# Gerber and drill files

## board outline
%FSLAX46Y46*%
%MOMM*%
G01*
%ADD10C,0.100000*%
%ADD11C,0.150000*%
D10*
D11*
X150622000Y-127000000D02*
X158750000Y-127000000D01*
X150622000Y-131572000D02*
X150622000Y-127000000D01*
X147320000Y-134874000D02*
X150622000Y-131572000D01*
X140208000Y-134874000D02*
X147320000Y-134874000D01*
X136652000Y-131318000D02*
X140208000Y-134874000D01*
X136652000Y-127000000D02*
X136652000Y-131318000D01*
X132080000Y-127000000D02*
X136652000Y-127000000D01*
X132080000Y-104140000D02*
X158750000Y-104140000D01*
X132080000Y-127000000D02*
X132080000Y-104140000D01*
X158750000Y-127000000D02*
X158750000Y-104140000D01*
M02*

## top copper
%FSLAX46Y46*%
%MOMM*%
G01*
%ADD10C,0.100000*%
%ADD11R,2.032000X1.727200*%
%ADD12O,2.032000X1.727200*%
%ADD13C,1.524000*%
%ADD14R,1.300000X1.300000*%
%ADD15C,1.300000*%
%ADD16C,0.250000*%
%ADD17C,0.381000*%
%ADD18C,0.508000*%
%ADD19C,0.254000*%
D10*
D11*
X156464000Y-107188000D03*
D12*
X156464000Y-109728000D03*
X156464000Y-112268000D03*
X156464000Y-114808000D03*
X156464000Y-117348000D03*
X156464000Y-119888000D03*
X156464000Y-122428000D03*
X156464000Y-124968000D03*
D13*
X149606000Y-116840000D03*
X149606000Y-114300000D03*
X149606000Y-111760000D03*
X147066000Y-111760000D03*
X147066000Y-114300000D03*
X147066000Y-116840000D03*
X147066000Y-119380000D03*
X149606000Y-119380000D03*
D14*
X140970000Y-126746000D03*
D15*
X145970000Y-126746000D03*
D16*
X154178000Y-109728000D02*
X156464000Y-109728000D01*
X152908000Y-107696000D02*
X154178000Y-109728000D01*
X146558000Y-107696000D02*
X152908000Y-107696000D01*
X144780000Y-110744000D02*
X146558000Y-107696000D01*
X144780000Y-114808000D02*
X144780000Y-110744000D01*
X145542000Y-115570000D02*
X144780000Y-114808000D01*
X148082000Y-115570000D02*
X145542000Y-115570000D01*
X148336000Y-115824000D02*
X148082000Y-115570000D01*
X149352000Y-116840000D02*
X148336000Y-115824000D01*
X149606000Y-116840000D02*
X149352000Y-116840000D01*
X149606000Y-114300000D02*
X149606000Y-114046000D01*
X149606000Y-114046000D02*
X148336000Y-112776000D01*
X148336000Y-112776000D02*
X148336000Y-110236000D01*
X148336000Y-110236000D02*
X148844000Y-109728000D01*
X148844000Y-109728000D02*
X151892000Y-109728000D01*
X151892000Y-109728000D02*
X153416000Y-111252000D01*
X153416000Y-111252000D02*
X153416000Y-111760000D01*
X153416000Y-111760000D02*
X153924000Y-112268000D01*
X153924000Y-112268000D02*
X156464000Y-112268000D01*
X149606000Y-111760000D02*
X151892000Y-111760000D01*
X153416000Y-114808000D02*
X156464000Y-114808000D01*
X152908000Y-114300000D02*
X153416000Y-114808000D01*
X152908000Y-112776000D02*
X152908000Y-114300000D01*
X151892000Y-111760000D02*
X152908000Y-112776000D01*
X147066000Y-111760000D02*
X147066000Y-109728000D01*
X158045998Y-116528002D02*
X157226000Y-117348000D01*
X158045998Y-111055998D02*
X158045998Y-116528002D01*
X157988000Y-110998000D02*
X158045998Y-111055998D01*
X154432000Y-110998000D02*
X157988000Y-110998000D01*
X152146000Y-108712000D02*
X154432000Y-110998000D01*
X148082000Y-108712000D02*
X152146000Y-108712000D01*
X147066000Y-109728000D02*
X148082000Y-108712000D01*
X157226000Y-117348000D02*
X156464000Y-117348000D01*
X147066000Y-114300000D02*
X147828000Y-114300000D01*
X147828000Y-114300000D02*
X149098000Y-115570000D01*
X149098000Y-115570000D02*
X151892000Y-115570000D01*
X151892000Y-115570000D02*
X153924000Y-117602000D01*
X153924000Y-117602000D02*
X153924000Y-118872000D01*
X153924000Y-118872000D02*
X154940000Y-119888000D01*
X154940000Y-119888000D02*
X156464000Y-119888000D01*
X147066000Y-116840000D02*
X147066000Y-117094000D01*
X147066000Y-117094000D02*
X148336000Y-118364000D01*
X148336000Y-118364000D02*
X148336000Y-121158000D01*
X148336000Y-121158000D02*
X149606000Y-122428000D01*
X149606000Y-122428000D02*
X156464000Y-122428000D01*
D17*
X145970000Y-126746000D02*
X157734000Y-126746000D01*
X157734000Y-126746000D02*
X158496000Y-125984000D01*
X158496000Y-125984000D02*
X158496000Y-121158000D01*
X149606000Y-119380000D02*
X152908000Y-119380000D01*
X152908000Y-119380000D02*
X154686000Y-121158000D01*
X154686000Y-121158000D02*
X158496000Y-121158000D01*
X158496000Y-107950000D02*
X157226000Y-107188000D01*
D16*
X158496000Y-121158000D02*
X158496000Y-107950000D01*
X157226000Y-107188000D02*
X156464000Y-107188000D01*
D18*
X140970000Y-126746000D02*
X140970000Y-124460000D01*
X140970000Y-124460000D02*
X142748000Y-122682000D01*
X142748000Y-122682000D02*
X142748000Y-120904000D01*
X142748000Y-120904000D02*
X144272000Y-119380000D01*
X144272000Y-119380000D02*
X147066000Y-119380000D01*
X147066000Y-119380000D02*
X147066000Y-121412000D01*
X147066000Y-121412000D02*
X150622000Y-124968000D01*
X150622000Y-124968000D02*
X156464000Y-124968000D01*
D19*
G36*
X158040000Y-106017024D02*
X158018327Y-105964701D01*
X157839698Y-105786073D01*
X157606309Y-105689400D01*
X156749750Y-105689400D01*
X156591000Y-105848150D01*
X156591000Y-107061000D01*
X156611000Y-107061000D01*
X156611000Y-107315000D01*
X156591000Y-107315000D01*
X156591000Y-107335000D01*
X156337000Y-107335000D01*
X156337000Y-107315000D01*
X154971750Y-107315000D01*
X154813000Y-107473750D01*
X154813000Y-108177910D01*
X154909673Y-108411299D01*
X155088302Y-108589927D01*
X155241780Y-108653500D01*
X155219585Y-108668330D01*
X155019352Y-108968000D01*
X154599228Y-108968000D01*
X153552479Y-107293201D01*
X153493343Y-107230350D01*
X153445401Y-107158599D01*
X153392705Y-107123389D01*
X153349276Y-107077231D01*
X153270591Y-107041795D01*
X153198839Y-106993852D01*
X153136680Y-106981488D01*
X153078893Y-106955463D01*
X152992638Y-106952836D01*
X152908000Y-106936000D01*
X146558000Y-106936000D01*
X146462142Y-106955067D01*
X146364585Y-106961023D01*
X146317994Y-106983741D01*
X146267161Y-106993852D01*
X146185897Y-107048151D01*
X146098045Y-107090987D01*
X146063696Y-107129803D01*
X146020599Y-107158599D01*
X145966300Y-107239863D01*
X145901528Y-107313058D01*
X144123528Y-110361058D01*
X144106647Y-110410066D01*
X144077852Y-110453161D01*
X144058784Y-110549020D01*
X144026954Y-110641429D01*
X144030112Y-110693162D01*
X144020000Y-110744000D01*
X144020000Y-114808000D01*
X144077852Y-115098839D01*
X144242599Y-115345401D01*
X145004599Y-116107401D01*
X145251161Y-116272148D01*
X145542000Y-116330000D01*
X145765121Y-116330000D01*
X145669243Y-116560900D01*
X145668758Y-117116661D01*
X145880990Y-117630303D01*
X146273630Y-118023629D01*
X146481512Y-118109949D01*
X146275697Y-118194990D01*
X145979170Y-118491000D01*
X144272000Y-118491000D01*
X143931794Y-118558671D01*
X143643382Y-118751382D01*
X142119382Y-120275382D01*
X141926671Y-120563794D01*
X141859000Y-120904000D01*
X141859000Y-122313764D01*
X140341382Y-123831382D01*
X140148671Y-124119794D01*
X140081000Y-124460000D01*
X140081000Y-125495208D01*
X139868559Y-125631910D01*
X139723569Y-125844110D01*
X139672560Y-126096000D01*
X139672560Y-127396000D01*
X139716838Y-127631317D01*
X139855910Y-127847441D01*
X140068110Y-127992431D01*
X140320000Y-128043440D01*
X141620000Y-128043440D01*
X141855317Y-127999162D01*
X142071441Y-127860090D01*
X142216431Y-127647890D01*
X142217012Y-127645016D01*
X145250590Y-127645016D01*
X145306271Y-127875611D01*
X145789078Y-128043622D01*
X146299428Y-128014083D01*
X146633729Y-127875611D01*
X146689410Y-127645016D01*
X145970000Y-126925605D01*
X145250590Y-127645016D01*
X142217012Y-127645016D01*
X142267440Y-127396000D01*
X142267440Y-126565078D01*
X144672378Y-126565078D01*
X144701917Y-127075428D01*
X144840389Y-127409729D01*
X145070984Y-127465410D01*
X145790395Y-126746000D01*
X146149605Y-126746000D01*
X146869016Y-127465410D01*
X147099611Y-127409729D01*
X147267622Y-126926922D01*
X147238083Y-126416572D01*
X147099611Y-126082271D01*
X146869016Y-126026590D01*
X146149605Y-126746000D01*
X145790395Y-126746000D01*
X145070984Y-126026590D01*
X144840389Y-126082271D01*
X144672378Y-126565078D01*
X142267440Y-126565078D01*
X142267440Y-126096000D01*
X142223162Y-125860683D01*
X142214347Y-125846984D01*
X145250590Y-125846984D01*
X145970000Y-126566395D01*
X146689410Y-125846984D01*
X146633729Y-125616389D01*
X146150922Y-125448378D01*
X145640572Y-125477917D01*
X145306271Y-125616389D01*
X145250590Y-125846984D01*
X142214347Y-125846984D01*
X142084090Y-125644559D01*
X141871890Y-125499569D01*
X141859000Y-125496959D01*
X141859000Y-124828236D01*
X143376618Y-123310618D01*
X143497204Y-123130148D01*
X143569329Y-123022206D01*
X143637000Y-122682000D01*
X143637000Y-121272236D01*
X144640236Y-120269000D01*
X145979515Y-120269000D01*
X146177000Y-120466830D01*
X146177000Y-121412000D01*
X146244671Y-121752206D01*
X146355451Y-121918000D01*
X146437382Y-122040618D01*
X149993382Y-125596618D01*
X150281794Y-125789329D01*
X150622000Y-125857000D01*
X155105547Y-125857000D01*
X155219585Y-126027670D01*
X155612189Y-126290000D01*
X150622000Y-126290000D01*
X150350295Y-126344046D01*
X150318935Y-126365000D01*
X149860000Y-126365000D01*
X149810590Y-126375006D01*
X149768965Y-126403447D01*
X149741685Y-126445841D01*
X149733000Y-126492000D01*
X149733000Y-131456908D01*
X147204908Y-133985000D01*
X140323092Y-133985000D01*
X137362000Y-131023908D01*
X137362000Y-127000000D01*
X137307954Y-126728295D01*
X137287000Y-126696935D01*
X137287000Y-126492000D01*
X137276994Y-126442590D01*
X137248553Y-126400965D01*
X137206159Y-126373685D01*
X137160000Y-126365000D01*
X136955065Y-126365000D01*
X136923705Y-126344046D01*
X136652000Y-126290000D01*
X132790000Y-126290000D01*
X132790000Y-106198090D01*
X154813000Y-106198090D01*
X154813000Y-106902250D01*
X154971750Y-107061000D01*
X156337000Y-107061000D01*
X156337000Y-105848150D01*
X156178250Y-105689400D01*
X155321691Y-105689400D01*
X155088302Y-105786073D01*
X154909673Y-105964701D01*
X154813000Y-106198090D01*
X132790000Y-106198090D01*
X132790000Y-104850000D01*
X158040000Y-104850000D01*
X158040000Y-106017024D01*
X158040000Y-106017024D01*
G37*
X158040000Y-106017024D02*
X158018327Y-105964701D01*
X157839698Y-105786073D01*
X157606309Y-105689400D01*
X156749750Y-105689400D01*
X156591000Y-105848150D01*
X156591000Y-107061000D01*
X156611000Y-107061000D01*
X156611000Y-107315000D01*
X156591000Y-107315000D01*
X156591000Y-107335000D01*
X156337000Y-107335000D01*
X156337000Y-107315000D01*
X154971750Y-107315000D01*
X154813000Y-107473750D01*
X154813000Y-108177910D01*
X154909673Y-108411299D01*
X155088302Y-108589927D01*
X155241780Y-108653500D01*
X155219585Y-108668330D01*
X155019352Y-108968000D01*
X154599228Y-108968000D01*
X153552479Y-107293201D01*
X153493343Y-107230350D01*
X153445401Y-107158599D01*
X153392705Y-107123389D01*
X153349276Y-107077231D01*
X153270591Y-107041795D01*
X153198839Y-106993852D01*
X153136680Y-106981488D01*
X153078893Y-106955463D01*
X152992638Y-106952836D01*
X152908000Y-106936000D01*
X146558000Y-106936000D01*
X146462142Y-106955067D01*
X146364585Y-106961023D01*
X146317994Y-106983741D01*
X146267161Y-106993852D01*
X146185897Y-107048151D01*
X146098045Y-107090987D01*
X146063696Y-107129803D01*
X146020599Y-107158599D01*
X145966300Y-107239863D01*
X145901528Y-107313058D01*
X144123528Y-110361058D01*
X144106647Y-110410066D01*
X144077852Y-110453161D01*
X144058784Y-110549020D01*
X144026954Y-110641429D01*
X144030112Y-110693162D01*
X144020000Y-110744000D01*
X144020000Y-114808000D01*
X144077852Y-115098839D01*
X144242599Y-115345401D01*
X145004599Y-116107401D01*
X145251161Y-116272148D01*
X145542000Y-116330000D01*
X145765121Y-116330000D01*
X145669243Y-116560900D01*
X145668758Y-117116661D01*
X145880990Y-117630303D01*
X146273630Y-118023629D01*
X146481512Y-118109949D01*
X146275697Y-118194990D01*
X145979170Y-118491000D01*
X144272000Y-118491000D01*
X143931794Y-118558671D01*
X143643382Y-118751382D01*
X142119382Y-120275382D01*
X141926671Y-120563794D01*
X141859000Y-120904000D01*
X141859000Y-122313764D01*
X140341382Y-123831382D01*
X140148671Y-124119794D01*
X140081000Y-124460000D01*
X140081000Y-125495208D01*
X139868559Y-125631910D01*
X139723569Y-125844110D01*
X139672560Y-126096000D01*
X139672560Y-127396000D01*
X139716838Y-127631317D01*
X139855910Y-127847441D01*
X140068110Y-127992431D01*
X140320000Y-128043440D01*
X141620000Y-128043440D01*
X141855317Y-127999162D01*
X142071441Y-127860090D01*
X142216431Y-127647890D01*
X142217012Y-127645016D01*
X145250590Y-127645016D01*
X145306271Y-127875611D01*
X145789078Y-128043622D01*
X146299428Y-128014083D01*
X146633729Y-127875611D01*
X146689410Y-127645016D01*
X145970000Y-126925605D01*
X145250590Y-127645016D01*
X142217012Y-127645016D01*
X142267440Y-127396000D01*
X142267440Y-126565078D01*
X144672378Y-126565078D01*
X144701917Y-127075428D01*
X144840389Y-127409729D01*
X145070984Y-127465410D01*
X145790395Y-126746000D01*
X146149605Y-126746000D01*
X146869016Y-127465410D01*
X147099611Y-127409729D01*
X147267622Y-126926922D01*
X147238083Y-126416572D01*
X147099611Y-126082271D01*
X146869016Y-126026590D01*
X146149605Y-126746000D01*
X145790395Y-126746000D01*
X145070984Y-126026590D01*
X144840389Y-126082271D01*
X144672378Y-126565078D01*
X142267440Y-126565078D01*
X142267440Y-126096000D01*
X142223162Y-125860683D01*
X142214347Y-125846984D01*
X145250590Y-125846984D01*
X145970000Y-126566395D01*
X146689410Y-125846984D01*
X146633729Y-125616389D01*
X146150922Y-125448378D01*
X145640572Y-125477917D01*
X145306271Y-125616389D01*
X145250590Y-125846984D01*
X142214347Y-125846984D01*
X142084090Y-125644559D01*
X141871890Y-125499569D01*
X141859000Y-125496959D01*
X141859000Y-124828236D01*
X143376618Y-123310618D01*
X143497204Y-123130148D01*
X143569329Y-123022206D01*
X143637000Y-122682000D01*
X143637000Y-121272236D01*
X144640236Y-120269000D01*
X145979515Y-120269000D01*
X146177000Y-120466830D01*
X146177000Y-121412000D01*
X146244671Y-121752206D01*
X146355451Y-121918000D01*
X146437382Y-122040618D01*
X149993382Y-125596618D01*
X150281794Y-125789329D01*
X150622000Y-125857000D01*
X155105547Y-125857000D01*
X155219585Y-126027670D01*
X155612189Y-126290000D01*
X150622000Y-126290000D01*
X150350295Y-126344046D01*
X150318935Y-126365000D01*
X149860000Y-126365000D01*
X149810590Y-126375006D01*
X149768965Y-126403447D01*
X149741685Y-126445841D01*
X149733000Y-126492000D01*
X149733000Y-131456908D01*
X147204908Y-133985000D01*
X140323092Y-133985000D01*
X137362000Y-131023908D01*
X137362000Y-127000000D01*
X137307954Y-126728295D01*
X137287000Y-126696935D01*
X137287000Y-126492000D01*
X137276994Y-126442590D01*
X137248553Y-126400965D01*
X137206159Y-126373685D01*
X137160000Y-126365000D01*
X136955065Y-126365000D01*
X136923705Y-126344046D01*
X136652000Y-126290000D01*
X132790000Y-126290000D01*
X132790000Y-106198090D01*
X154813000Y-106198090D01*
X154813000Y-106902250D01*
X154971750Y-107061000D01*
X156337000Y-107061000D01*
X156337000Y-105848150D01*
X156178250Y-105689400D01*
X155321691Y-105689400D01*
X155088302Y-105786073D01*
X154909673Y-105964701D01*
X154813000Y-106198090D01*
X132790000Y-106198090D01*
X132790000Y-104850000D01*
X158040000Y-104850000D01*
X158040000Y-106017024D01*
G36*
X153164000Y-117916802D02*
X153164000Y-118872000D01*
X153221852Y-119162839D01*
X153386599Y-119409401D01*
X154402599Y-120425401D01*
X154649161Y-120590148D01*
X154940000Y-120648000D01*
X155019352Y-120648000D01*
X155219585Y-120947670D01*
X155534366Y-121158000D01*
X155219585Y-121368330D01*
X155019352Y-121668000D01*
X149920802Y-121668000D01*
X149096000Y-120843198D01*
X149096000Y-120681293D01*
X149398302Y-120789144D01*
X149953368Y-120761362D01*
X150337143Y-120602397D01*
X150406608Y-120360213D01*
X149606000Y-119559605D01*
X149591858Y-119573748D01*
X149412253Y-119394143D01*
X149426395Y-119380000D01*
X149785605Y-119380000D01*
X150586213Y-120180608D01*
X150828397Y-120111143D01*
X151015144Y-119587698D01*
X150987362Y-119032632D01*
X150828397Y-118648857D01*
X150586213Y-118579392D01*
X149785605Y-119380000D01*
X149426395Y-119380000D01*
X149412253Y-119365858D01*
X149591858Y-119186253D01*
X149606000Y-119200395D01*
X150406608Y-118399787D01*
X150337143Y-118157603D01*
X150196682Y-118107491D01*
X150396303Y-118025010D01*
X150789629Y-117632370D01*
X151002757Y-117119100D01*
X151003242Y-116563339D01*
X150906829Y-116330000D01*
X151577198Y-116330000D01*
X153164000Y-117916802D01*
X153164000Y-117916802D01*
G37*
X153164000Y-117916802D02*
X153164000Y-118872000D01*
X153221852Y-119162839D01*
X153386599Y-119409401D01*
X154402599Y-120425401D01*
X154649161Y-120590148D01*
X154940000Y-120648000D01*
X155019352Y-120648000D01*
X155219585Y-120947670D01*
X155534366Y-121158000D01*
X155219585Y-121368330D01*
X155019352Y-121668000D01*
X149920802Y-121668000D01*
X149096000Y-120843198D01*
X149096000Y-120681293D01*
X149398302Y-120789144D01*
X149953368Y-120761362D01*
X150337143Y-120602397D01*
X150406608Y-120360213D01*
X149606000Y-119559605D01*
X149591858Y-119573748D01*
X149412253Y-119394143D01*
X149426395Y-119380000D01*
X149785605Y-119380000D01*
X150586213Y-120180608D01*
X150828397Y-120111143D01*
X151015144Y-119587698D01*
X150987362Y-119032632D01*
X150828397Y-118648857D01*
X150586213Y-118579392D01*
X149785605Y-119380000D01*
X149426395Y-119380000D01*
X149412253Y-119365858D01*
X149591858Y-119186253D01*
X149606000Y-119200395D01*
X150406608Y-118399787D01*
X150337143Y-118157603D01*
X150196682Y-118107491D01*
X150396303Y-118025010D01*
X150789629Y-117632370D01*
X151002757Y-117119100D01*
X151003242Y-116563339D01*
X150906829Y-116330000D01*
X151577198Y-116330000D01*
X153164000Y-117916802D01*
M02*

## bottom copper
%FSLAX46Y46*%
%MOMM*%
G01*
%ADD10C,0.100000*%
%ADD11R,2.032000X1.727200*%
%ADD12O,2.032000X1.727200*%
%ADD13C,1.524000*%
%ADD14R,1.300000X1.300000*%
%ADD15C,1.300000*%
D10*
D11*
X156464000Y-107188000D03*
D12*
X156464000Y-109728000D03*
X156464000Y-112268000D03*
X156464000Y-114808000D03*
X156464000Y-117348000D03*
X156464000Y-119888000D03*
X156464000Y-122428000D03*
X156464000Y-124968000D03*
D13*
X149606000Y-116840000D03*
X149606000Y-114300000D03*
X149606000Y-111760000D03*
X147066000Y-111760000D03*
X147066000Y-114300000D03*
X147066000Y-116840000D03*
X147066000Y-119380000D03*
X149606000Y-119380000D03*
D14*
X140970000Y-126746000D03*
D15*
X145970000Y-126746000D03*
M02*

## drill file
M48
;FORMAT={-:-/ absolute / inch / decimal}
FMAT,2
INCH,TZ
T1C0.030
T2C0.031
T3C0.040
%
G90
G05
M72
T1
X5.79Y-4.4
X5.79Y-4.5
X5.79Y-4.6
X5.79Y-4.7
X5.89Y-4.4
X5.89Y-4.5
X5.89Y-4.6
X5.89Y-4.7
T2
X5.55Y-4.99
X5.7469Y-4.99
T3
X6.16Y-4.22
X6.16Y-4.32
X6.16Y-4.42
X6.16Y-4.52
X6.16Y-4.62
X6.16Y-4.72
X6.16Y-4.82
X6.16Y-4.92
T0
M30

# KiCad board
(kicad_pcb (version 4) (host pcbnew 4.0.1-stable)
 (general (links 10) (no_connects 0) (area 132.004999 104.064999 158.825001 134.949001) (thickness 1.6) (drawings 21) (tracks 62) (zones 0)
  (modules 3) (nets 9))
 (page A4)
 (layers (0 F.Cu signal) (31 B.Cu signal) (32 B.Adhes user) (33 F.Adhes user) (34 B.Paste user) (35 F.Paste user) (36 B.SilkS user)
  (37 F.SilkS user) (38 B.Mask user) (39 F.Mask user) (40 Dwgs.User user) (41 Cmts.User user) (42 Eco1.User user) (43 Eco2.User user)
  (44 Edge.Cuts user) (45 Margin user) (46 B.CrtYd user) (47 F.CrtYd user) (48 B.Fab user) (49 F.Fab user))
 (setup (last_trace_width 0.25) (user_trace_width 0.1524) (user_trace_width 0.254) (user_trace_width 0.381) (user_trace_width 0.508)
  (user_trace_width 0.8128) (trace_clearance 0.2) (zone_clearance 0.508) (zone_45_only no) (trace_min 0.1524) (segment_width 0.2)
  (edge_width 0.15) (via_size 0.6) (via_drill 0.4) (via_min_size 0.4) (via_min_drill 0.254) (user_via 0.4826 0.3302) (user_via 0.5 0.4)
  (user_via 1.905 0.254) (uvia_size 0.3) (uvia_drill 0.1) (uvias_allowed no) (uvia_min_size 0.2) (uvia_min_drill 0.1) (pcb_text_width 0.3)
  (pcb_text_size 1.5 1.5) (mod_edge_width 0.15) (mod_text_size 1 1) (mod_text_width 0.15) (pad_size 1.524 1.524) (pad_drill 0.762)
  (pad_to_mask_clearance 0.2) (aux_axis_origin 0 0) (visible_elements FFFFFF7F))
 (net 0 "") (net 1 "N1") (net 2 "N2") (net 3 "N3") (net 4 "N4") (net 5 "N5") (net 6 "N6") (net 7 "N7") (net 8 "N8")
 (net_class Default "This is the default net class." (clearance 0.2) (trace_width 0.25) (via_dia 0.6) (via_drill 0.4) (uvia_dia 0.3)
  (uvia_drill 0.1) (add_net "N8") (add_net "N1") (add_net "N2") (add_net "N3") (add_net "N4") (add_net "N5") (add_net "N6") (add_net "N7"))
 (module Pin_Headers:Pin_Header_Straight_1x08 (layer F.Cu) (at 156.464 107.188)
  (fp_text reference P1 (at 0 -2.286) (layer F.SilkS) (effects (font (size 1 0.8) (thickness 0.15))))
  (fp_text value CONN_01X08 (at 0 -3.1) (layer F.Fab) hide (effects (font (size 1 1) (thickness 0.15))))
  (pad 1 thru_hole rect (at 0 0) (size 2.032 1.7272) (drill 1.016) (layers *.Cu *.Mask F.SilkS) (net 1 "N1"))
  (pad 2 thru_hole oval (at 0 2.54) (size 2.032 1.7272) (drill 1.016) (layers *.Cu *.Mask F.SilkS) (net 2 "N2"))
  (pad 3 thru_hole oval (at 0 5.08) (size 2.032 1.7272) (drill 1.016) (layers *.Cu *.Mask F.SilkS) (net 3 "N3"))
  (pad 4 thru_hole oval (at 0 7.62) (size 2.032 1.7272) (drill 1.016) (layers *.Cu *.Mask F.SilkS) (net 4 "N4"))
  (pad 5 thru_hole oval (at 0 10.16) (size 2.032 1.7272) (drill 1.016) (layers *.Cu *.Mask F.SilkS) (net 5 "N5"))
  (pad 6 thru_hole oval (at 0 12.7) (size 2.032 1.7272) (drill 1.016) (layers *.Cu *.Mask F.SilkS) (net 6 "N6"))
  (pad 7 thru_hole oval (at 0 15.24) (size 2.032 1.7272) (drill 1.016) (layers *.Cu *.Mask F.SilkS) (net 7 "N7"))
  (pad 8 thru_hole oval (at 0 17.78) (size 2.032 1.7272) (drill 1.016) (layers *.Cu *.Mask F.SilkS) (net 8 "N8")))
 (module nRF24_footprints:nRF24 (layer F.Cu) (at 139.446 119.38)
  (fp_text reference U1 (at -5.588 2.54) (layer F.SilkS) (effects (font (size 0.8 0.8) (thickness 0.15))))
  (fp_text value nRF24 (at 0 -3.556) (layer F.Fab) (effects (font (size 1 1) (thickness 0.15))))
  (pad 1 thru_hole circle (at 10.16 -2.54) (size 1.524 1.524) (drill 0.762) (layers *.Cu *.Mask F.SilkS) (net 2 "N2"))
  (pad 2 thru_hole circle (at 10.16 -5.08) (size 1.524 1.524) (drill 0.762) (layers *.Cu *.Mask F.SilkS) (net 3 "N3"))
  (pad 3 thru_hole circle (at 10.16 -7.62) (size 1.524 1.524) (drill 0.762) (layers *.Cu *.Mask F.SilkS) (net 4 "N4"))
  (pad 4 thru_hole circle (at 7.62 -7.62) (size 1.524 1.524) (drill 0.762) (layers *.Cu *.Mask F.SilkS) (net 5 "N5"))
  (pad 5 thru_hole circle (at 7.62 -5.08) (size 1.524 1.524) (drill 0.762) (layers *.Cu *.Mask F.SilkS) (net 6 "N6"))
  (pad 6 thru_hole circle (at 7.62 -2.54) (size 1.524 1.524) (drill 0.762) (layers *.Cu *.Mask F.SilkS) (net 7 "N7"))
  (pad 7 thru_hole circle (at 7.62 0) (size 1.524 1.524) (drill 0.762) (layers *.Cu *.Mask F.SilkS) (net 8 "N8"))
  (pad 0 thru_hole circle (at 10.16 0) (size 1.524 1.524) (drill 0.762) (layers *.Cu *.Mask F.SilkS) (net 1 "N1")))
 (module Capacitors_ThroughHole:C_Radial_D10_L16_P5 (layer F.Cu) (at 140.97 126.746)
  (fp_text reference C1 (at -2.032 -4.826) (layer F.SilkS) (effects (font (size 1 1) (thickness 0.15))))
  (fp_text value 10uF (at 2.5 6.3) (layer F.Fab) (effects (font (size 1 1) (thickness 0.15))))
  (pad 1 thru_hole rect (at 0 0) (size 1.3 1.3) (drill 0.8) (layers *.Cu *.Mask F.SilkS) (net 8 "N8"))
  (pad 2 thru_hole circle (at 5 0) (size 1.3 1.3) (drill 0.8) (layers *.Cu *.Mask F.SilkS) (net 1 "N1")))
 (gr_line (start 150.622 127) (end 158.75 127) (angle 90) (layer Edge.Cuts) (width 0.15))
 (gr_line (start 150.622 131.572) (end 150.622 127) (angle 90) (layer Edge.Cuts) (width 0.15))
 (gr_line (start 147.32 134.874) (end 150.622 131.572) (angle 90) (layer Edge.Cuts) (width 0.15))
 (gr_line (start 140.208 134.874) (end 147.32 134.874) (angle 90) (layer Edge.Cuts) (width 0.15))
 (gr_line (start 136.652 131.318) (end 140.208 134.874) (angle 90) (layer Edge.Cuts) (width 0.15))
 (gr_line (start 136.652 127) (end 136.652 131.318) (angle 90) (layer Edge.Cuts) (width 0.15))
 (gr_line (start 132.08 127) (end 136.652 127) (angle 90) (layer Edge.Cuts) (width 0.15))
 (gr_line (start 132.08 104.14) (end 158.75 104.14) (angle 90) (layer Edge.Cuts) (width 0.15))
 (gr_line (start 132.08 127) (end 132.08 104.14) (angle 90) (layer Edge.Cuts) (width 0.15))
 (gr_line (start 158.75 127) (end 158.75 104.14) (angle 90) (layer Edge.Cuts) (width 0.15))
 (segment (start 154.178 109.728) (end 156.464 109.728) (width 0.25) (layer F.Cu) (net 2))
 (segment (start 152.908 107.696) (end 154.178 109.728) (width 0.25) (layer F.Cu) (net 2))
 (segment (start 146.558 107.696) (end 152.908 107.696) (width 0.25) (layer F.Cu) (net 2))
 (segment (start 144.78 110.744) (end 146.558 107.696) (width 0.25) (layer F.Cu) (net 2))
 (segment (start 144.78 114.808) (end 144.78 110.744) (width 0.25) (layer F.Cu) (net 2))
 (segment (start 145.542 115.57) (end 144.78 114.808) (width 0.25) (layer F.Cu) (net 2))
 (segment (start 148.082 115.57) (end 145.542 115.57) (width 0.25) (layer F.Cu) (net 2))
 (segment (start 148.336 115.824) (end 148.082 115.57) (width 0.25) (layer F.Cu) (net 2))
 (segment (start 149.352 116.84) (end 148.336 115.824) (width 0.25) (layer F.Cu) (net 2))
 (segment (start 149.606 116.84) (end 149.352 116.84) (width 0.25) (layer F.Cu) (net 2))
 (segment (start 149.606 114.3) (end 149.606 114.046) (width 0.25) (layer F.Cu) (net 3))
 (segment (start 149.606 114.046) (end 148.336 112.776) (width 0.25) (layer F.Cu) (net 3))
 (segment (start 148.336 112.776) (end 148.336 110.236) (width 0.25) (layer F.Cu) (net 3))
 (segment (start 148.336 110.236) (end 148.844 109.728) (width 0.25) (layer F.Cu) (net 3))
 (segment (start 148.844 109.728) (end 151.892 109.728) (width 0.25) (layer F.Cu) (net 3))
 (segment (start 151.892 109.728) (end 153.416 111.252) (width 0.25) (layer F.Cu) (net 3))
 (segment (start 153.416 111.252) (end 153.416 111.76) (width 0.25) (layer F.Cu) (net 3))
 (segment (start 153.416 111.76) (end 153.924 112.268) (width 0.25) (layer F.Cu) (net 3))
 (segment (start 153.924 112.268) (end 156.464 112.268) (width 0.25) (layer F.Cu) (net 3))
 (segment (start 149.606 111.76) (end 151.892 111.76) (width 0.25) (layer F.Cu) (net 4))
 (segment (start 153.416 114.808) (end 156.464 114.808) (width 0.25) (layer F.Cu) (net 4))
 (segment (start 152.908 114.3) (end 153.416 114.808) (width 0.25) (layer F.Cu) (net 4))
 (segment (start 152.908 112.776) (end 152.908 114.3) (width 0.25) (layer F.Cu) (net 4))
 (segment (start 151.892 111.76) (end 152.908 112.776) (width 0.25) (layer F.Cu) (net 4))
 (segment (start 147.066 111.76) (end 147.066 109.728) (width 0.25) (layer F.Cu) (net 5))
 (segment (start 158.045998 116.528002) (end 157.226 117.348) (width 0.25) (layer F.Cu) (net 5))
 (segment (start 158.045998 111.055998) (end 158.045998 116.528002) (width 0.25) (layer F.Cu) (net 5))
 (segment (start 157.988 110.998) (end 158.045998 111.055998) (width 0.25) (layer F.Cu) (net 5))
 (segment (start 154.432 110.998) (end 157.988 110.998) (width 0.25) (layer F.Cu) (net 5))
 (segment (start 152.146 108.712) (end 154.432 110.998) (width 0.25) (layer F.Cu) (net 5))
 (segment (start 148.082 108.712) (end 152.146 108.712) (width 0.25) (layer F.Cu) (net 5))
 (segment (start 147.066 109.728) (end 148.082 108.712) (width 0.25) (layer F.Cu) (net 5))
 (segment (start 157.226 117.348) (end 156.464 117.348) (width 0.25) (layer F.Cu) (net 5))
 (segment (start 147.066 114.3) (end 147.828 114.3) (width 0.25) (layer F.Cu) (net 6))
 (segment (start 147.828 114.3) (end 149.098 115.57) (width 0.25) (layer F.Cu) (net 6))
 (segment (start 149.098 115.57) (end 151.892 115.57) (width 0.25) (layer F.Cu) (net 6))
 (segment (start 151.892 115.57) (end 153.924 117.602) (width 0.25) (layer F.Cu) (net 6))
 (segment (start 153.924 117.602) (end 153.924 118.872) (width 0.25) (layer F.Cu) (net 6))
 (segment (start 153.924 118.872) (end 154.94 119.888) (width 0.25) (layer F.Cu) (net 6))
 (segment (start 154.94 119.888) (end 156.464 119.888) (width 0.25) (layer F.Cu) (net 6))
 (segment (start 147.066 116.84) (end 147.066 117.094) (width 0.25) (layer F.Cu) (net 7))
 (segment (start 147.066 117.094) (end 148.336 118.364) (width 0.25) (layer F.Cu) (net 7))
 (segment (start 148.336 118.364) (end 148.336 121.158) (width 0.25) (layer F.Cu) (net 7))
 (segment (start 148.336 121.158) (end 149.606 122.428) (width 0.25) (layer F.Cu) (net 7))
 (segment (start 149.606 122.428) (end 156.464 122.428) (width 0.25) (layer F.Cu) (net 7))
 (segment (start 145.97 126.746) (end 157.734 126.746) (width 0.381) (layer F.Cu) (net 1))
 (segment (start 157.734 126.746) (end 158.496 125.984) (width 0.381) (layer F.Cu) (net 1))
 (segment (start 158.496 125.984) (end 158.496 121.158) (width 0.381) (layer F.Cu) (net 1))
 (segment (start 149.606 119.38) (end 152.908 119.38) (width 0.381) (layer F.Cu) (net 1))
 (segment (start 152.908 119.38) (end 154.686 121.158) (width 0.381) (layer F.Cu) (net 1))
 (segment (start 154.686 121.158) (end 158.496 121.158) (width 0.381) (layer F.Cu) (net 1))
 (segment (start 158.496 107.95) (end 157.226 107.188) (width 0.381) (layer F.Cu) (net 1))
 (segment (start 158.496 121.158) (end 158.496 107.95) (width 0.25) (layer F.Cu) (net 1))
 (segment (start 157.226 107.188) (end 156.464 107.188) (width 0.25) (layer F.Cu) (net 1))
 (segment (start 140.97 126.746) (end 140.97 124.46) (width 0.508) (layer F.Cu) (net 8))
 (segment (start 140.97 124.46) (end 142.748 122.682) (width 0.508) (layer F.Cu) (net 8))
 (segment (start 142.748 122.682) (end 142.748 120.904) (width 0.508) (layer F.Cu) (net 8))
 (segment (start 142.748 120.904) (end 144.272 119.38) (width 0.508) (layer F.Cu) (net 8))
 (segment (start 144.272 119.38) (end 147.066 119.38) (width 0.508) (layer F.Cu) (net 8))
 (segment (start 147.066 119.38) (end 147.066 121.412) (width 0.508) (layer F.Cu) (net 8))
 (segment (start 147.066 121.412) (end 150.622 124.968) (width 0.508) (layer F.Cu) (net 8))
 (segment (start 150.622 124.968) (end 156.464 124.968) (width 0.508) (layer F.Cu) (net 8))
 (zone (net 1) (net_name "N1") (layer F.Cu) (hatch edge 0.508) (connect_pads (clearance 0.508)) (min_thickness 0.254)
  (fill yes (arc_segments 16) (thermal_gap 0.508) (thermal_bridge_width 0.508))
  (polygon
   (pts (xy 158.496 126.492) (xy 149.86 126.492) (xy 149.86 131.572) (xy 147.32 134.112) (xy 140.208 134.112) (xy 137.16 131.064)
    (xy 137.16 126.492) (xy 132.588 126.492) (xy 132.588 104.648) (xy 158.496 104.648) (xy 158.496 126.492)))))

